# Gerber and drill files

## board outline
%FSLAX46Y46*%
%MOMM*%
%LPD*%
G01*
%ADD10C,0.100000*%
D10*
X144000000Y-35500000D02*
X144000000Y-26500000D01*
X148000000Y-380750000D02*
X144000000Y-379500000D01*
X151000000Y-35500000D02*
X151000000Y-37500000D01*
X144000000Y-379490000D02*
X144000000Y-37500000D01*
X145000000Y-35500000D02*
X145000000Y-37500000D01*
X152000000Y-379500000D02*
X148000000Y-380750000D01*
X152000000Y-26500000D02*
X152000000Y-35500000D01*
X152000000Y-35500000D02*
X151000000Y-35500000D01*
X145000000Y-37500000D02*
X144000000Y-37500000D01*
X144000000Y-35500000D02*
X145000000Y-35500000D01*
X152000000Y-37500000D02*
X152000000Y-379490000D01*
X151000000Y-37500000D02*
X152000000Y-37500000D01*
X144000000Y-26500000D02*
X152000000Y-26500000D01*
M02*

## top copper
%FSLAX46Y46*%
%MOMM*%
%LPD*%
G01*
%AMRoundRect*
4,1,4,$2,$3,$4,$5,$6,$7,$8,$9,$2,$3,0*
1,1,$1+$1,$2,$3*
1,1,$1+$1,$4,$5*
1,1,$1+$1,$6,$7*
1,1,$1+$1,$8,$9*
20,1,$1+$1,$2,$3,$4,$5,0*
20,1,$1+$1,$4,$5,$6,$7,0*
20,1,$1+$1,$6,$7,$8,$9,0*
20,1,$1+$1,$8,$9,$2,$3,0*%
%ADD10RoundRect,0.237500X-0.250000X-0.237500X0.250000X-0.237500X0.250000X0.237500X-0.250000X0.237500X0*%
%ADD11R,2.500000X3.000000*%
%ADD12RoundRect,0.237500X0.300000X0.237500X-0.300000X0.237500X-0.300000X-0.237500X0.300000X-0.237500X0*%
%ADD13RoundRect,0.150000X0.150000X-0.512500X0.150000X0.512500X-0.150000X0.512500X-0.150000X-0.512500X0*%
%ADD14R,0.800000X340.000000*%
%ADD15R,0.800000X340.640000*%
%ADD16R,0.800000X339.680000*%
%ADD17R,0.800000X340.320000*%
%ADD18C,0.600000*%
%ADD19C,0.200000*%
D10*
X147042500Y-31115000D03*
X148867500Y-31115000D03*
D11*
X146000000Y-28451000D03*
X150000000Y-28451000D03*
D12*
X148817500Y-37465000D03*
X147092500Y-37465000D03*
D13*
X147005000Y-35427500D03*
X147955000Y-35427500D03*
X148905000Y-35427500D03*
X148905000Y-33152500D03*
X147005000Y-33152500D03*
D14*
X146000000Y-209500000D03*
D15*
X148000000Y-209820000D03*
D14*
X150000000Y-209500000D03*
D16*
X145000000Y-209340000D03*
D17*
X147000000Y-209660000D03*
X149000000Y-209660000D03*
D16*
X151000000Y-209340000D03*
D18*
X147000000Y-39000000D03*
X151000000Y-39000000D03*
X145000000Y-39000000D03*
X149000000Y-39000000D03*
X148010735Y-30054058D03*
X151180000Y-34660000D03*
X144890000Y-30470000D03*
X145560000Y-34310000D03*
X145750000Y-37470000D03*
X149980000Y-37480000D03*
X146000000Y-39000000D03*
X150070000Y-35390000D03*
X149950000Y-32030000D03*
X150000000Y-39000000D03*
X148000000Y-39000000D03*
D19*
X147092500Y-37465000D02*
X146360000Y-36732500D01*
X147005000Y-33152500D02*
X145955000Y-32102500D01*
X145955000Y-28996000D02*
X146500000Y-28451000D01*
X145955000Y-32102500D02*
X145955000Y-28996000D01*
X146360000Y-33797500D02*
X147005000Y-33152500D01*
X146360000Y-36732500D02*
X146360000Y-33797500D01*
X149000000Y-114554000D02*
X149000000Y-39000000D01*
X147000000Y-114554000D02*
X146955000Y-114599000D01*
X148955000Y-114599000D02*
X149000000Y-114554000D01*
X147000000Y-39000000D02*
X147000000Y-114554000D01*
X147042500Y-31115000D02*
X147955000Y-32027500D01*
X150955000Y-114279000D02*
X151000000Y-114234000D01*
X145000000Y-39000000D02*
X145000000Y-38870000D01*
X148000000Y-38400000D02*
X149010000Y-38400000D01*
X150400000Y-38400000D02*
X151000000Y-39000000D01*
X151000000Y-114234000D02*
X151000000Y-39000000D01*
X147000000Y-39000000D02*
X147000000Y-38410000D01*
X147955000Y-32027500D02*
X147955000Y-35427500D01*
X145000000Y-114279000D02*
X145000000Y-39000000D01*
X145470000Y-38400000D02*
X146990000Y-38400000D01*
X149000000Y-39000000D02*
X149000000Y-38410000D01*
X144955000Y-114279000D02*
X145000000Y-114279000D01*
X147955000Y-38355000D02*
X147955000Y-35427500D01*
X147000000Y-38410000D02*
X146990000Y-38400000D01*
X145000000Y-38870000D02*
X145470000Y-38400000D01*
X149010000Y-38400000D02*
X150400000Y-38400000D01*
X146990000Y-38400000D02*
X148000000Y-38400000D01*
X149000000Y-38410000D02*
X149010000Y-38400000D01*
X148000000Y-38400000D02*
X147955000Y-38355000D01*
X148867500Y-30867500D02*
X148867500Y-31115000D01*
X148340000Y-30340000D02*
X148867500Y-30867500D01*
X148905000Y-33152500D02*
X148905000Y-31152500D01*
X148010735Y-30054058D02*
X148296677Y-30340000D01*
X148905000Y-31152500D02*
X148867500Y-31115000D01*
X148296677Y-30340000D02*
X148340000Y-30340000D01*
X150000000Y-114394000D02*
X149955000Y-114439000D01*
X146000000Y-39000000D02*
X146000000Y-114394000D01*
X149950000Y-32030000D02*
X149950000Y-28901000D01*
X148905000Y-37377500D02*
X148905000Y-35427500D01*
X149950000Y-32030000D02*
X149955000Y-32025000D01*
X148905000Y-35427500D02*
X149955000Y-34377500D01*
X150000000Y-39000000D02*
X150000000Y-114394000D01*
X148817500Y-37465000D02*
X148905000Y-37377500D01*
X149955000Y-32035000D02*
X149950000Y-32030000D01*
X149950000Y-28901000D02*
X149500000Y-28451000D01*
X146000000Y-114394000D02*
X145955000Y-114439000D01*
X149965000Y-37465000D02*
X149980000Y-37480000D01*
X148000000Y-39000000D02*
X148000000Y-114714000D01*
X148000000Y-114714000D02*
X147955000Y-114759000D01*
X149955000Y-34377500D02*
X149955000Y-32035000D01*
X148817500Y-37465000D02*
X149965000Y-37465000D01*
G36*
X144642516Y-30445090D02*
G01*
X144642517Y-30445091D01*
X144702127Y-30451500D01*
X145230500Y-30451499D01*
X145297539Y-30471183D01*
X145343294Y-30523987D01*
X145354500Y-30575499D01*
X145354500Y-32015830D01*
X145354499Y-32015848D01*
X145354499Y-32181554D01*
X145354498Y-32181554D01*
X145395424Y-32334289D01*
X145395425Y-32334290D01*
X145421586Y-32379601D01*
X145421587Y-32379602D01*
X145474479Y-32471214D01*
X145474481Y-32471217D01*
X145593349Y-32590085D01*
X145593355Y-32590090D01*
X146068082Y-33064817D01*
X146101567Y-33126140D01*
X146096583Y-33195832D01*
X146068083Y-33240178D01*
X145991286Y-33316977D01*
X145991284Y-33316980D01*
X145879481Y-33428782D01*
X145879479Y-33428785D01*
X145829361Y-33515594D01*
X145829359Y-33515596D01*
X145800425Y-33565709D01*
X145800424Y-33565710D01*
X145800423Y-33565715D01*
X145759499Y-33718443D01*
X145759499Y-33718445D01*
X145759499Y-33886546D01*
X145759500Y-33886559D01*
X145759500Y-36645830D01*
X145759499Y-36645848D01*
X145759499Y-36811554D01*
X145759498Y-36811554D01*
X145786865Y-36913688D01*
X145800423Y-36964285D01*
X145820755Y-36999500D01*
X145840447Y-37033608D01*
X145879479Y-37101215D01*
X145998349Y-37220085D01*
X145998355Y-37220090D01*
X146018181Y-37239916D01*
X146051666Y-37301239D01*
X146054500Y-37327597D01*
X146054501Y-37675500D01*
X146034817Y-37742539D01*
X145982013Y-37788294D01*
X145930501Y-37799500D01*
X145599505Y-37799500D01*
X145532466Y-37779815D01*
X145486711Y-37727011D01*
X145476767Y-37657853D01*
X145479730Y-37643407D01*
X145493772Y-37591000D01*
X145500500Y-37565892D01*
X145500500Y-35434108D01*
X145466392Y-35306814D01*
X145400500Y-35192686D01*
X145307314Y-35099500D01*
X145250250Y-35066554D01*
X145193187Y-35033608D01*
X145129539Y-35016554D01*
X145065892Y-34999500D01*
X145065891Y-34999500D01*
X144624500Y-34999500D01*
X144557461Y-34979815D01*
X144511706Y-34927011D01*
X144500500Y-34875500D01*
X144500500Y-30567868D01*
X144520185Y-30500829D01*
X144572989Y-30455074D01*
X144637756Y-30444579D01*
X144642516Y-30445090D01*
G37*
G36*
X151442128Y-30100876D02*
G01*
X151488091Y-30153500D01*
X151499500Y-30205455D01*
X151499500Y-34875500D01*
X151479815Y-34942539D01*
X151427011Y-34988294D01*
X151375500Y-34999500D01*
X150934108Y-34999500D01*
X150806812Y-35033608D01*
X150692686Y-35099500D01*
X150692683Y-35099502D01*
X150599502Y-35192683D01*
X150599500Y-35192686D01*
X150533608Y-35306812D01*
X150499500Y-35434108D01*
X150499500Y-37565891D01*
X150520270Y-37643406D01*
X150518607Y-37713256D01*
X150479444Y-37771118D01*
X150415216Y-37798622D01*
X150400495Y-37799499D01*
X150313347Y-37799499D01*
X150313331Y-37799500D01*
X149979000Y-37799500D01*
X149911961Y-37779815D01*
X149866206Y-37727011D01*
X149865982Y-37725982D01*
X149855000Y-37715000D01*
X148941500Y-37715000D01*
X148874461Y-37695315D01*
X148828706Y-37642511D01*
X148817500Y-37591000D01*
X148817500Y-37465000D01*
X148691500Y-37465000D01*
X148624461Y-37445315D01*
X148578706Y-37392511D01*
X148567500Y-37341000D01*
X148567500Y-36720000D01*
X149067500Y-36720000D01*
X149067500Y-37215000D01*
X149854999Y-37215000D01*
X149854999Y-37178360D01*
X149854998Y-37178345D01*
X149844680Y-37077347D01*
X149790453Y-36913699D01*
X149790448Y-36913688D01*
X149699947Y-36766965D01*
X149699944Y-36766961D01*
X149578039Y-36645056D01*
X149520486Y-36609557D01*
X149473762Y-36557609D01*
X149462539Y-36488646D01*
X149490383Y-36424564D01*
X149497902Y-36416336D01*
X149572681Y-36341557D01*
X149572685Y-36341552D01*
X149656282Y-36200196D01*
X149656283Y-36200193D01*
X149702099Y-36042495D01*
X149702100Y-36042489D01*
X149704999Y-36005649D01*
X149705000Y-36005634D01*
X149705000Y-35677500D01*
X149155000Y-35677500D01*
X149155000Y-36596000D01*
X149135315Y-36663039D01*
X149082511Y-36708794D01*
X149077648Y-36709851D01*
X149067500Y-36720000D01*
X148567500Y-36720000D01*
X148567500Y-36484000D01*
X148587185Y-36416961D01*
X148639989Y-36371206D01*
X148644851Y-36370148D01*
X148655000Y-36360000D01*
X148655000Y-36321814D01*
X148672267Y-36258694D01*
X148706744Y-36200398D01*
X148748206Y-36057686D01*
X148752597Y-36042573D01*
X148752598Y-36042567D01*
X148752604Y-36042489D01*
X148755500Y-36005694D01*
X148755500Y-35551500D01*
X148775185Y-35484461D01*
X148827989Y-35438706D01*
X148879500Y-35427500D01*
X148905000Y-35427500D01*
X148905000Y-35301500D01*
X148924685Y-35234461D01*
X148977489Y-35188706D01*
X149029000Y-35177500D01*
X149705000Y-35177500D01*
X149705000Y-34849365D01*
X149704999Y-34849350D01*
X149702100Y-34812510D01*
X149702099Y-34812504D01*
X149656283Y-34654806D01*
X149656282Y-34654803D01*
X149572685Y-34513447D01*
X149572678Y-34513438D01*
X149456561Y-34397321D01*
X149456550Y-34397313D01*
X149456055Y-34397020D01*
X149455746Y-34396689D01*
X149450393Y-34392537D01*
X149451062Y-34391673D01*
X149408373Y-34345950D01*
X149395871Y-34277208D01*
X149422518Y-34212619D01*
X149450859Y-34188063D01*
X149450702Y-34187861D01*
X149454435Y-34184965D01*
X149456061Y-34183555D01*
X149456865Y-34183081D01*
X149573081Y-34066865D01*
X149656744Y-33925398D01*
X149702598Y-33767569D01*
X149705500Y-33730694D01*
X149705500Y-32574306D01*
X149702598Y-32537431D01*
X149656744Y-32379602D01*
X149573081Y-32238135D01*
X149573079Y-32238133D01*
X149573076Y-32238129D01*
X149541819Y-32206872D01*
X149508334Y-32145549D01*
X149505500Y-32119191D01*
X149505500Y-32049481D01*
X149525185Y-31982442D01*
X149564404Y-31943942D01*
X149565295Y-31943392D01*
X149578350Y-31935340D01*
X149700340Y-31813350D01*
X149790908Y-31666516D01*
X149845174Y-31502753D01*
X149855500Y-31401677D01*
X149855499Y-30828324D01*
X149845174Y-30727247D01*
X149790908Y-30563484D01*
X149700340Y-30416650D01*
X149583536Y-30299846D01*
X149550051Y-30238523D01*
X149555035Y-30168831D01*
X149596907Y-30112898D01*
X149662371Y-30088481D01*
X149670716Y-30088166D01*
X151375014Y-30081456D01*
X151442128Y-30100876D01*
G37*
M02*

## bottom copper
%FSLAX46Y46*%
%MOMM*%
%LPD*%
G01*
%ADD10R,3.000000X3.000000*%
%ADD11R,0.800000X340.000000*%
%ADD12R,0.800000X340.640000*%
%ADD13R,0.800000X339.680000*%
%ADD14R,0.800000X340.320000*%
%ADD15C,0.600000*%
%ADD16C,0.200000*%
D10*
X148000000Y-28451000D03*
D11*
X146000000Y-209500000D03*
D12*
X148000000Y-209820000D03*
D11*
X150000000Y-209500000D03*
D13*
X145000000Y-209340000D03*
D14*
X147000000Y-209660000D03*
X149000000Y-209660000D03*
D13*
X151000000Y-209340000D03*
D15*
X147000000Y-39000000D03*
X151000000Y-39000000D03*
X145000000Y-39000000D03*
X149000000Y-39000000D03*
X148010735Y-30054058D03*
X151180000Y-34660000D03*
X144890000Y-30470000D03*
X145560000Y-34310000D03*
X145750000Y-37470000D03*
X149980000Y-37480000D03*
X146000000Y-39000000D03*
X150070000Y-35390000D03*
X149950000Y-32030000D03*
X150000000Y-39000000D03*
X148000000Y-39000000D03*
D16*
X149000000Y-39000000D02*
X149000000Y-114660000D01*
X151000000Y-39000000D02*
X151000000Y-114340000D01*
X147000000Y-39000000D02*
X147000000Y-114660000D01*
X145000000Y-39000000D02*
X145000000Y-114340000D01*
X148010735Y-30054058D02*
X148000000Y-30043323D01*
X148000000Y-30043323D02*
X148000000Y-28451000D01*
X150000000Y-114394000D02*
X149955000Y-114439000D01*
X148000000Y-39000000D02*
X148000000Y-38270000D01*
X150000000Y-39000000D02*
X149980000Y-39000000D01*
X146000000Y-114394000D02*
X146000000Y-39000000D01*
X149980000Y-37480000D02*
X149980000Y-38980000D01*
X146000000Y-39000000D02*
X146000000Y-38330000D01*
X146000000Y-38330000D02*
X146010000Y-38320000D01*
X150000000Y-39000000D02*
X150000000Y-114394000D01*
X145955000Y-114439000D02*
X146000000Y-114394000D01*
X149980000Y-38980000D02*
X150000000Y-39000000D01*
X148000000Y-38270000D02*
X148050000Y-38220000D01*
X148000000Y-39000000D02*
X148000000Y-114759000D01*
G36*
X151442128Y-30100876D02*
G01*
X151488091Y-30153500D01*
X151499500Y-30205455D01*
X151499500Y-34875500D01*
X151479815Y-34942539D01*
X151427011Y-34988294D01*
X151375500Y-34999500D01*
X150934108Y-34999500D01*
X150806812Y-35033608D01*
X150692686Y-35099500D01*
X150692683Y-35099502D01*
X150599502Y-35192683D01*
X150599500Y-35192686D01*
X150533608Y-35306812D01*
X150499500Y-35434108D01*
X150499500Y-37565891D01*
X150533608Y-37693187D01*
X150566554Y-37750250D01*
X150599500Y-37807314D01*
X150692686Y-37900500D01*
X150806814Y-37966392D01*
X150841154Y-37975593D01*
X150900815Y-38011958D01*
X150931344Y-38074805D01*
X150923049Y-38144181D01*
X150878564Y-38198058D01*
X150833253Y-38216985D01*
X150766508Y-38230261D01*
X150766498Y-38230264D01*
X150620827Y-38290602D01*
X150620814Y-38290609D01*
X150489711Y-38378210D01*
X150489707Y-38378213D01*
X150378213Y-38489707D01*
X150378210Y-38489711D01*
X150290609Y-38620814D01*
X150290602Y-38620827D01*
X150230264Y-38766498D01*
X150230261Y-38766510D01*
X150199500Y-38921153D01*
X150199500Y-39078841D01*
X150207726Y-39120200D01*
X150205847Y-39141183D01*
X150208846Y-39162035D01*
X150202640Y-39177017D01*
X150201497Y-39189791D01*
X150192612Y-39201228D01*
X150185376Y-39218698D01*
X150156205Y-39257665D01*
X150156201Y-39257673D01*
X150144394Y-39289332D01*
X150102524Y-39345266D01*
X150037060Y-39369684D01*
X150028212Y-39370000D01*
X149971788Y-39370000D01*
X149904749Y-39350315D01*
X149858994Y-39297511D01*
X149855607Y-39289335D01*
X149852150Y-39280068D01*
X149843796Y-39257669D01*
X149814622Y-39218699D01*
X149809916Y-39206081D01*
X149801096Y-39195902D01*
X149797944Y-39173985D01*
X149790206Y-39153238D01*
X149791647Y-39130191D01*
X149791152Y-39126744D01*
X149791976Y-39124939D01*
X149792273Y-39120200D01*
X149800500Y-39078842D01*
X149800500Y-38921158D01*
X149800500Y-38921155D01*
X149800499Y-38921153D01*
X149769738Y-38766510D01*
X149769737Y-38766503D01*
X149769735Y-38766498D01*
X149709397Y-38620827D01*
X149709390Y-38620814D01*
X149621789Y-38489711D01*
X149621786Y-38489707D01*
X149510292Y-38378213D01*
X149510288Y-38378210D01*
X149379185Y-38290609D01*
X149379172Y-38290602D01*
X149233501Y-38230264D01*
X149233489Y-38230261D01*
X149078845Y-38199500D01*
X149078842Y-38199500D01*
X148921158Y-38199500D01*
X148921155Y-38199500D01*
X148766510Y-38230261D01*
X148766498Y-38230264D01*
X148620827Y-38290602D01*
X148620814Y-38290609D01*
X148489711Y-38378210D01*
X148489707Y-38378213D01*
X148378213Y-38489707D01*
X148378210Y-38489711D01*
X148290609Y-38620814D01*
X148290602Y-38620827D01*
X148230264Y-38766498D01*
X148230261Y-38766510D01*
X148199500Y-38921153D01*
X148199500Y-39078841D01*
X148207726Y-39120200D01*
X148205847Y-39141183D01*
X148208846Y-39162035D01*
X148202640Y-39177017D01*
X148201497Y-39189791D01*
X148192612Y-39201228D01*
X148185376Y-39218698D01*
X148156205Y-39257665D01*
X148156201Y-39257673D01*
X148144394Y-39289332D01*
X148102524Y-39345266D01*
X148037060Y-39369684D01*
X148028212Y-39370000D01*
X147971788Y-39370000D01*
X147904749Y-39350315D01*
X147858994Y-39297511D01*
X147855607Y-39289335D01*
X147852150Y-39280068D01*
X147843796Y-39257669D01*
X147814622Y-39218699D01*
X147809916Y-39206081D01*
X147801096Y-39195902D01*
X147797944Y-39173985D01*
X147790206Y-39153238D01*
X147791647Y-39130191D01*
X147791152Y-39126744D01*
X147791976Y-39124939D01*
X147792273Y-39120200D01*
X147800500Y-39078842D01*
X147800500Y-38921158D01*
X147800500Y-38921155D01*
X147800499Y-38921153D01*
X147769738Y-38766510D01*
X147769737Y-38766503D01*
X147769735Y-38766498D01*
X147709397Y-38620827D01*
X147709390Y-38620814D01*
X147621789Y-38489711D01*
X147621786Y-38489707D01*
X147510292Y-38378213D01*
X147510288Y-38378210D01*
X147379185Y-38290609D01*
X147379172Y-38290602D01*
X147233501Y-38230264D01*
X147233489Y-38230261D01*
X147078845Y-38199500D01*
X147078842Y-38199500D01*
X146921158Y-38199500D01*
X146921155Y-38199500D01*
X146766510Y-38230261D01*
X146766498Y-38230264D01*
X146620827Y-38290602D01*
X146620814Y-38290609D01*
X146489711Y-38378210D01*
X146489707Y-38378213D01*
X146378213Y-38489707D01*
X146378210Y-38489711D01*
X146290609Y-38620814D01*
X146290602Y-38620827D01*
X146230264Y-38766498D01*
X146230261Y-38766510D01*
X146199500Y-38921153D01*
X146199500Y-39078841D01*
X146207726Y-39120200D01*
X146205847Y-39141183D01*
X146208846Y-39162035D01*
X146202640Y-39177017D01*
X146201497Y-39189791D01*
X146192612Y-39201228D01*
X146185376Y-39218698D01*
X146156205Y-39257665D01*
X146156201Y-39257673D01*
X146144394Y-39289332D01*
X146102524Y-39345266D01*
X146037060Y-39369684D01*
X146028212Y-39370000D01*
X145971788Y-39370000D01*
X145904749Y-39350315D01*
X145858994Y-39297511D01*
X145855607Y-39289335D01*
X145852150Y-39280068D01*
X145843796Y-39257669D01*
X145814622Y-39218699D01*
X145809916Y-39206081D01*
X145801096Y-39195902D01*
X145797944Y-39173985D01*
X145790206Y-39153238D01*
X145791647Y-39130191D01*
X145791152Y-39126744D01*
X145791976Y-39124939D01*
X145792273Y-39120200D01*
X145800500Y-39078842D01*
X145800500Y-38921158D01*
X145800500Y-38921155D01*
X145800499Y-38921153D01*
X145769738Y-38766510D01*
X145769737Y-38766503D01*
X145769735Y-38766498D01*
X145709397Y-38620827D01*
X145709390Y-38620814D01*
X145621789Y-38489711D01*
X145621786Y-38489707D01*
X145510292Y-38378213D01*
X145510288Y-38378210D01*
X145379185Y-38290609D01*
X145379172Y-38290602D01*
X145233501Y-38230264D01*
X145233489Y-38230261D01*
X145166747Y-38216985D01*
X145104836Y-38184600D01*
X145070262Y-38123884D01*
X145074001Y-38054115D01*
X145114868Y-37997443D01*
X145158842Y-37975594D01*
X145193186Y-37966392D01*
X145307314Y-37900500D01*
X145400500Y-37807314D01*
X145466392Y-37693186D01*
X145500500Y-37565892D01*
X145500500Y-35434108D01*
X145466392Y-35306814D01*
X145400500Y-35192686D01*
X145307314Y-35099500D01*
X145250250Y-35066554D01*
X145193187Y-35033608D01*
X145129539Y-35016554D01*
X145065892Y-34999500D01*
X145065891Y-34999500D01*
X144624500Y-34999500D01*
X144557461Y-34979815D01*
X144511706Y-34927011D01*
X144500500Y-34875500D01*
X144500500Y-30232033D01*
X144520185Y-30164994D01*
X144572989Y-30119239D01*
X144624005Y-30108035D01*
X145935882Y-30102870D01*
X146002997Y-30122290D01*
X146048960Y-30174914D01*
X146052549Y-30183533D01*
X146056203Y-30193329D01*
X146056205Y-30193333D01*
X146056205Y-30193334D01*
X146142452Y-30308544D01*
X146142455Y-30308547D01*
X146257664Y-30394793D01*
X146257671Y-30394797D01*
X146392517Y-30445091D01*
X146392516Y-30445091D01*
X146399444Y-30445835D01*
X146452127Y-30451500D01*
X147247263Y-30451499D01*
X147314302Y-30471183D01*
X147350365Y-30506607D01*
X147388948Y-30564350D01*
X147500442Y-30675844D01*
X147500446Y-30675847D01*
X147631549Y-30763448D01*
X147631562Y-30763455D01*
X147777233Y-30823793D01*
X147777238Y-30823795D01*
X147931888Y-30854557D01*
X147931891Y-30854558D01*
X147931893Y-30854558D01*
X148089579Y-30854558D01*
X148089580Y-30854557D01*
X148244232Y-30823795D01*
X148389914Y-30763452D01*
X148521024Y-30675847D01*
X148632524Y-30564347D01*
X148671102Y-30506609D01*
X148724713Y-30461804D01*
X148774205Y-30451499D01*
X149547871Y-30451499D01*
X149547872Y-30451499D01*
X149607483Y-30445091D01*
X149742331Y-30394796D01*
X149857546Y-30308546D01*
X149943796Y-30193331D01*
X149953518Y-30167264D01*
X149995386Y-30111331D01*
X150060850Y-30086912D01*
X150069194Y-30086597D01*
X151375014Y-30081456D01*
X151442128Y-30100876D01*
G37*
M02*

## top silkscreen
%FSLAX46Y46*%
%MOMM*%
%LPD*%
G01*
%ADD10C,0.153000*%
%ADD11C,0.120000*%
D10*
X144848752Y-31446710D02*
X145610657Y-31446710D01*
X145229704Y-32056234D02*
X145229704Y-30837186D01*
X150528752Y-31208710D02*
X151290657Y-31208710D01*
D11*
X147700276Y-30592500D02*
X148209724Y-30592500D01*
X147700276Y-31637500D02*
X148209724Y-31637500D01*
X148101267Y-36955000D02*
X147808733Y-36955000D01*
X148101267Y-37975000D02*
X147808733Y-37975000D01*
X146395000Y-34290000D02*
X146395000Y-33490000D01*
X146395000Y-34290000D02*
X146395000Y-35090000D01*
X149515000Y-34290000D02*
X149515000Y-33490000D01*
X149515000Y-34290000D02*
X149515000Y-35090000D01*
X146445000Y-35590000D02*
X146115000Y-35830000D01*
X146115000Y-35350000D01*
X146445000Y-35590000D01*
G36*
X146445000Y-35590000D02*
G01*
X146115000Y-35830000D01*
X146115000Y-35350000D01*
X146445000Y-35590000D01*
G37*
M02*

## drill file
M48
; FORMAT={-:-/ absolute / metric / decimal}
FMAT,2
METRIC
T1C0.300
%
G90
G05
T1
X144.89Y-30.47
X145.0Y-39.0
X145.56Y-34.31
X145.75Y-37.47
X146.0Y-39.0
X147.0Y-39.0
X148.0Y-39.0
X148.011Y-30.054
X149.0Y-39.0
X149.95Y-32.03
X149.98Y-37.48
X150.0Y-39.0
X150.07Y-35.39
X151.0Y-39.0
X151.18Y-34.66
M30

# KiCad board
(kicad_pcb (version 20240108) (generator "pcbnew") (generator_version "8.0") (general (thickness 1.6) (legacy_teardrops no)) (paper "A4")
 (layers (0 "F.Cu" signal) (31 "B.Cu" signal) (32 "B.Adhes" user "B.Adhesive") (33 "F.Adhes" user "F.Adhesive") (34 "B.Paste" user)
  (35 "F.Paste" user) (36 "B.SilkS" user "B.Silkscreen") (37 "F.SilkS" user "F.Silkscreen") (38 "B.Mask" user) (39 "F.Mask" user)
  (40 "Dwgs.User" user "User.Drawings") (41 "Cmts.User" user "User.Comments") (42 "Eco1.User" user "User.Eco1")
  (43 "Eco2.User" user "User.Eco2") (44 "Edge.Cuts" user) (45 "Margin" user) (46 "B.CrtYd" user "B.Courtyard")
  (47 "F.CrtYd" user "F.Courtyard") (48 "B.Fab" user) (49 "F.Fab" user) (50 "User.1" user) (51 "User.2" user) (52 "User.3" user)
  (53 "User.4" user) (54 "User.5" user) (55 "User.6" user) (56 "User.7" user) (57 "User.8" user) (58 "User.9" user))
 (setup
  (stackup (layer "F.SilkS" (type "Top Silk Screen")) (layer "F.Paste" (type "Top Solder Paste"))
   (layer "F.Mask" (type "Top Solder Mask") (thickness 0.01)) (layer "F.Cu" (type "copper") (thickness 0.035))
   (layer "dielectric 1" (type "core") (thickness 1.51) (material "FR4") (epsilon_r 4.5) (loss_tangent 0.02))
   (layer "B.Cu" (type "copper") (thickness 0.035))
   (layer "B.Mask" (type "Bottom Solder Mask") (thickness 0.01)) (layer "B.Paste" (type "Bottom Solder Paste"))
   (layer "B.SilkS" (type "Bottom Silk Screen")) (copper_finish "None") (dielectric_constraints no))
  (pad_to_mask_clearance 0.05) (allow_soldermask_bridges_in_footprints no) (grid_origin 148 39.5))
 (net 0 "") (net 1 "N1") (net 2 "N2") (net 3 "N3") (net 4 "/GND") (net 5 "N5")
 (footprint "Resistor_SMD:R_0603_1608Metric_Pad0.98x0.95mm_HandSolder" (layer "F.Cu") (at 147.955 31.115)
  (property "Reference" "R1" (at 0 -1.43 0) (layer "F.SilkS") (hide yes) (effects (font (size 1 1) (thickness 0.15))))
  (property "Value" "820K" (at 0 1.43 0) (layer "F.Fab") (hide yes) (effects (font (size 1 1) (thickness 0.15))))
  (fp_line (start -0.254724 -0.5225) (end 0.254724 -0.5225) (stroke (width 0.12) (type solid)) (layer "F.SilkS"))
  (fp_line (start -0.254724 0.5225) (end 0.254724 0.5225) (stroke (width 0.12) (type solid)) (layer "F.SilkS"))
  (pad "1" smd roundrect (at -0.9125 0) (size 0.975 0.95) (layers "F.Cu" "F.Paste" "F.Mask") (roundrect_rratio 0.25) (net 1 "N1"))
  (pad "2" smd roundrect (at 0.9125 0) (size 0.975 0.95) (layers "F.Cu" "F.Paste" "F.Mask") (roundrect_rratio 0.25) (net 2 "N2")))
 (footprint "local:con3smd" (layer "F.Cu") (at 148 28.451)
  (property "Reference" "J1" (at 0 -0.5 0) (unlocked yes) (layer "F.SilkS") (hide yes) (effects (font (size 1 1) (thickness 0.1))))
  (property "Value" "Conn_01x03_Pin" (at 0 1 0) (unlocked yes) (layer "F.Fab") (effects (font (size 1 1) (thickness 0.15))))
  (pad "1" smd rect (at -2 0) (size 2.5 3) (layers "F.Cu" "F.Paste" "F.Mask") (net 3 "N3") (thermal_bridge_angle 45))
  (pad "2" smd rect (at 0 0) (size 3 3) (layers "B.Cu" "B.Paste" "B.Mask") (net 2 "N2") (thermal_bridge_angle 45))
  (pad "3" smd rect (at 2 0) (size 2.5 3) (layers "F.Cu" "F.Paste" "F.Mask") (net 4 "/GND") (thermal_bridge_angle 45)))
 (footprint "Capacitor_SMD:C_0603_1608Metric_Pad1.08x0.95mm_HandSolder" (layer "F.Cu") (at 147.955 37.465 180)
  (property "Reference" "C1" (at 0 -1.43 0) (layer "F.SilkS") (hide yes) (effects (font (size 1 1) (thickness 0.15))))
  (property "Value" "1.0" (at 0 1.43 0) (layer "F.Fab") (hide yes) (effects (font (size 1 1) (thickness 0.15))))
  (fp_line (start -0.146267 0.51) (end 0.146267 0.51) (stroke (width 0.12) (type solid)) (layer "F.SilkS"))
  (fp_line (start -0.146267 -0.51) (end 0.146267 -0.51) (stroke (width 0.12) (type solid)) (layer "F.SilkS"))
  (pad "1" smd roundrect (at -0.8625 0 180) (size 1.075 0.95) (layers "F.Cu" "F.Paste" "F.Mask") (roundrect_rratio 0.25) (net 4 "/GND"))
  (pad "2" smd roundrect (at 0.8625 0 180) (size 1.075 0.95) (layers "F.Cu" "F.Paste" "F.Mask") (roundrect_rratio 0.25) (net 3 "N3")))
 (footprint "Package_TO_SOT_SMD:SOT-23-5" (layer "F.Cu") (at 147.955 34.29 90)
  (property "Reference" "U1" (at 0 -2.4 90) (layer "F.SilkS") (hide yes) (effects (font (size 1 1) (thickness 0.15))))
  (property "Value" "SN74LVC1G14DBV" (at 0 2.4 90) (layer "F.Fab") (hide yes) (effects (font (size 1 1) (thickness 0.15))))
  (fp_line (start 0 -1.56) (end 0.8 -1.56) (stroke (width 0.12) (type solid)) (layer "F.SilkS"))
  (fp_line (start 0 -1.56) (end -0.8 -1.56) (stroke (width 0.12) (type solid)) (layer "F.SilkS"))
  (fp_line (start 0 1.56) (end 0.8 1.56) (stroke (width 0.12) (type solid)) (layer "F.SilkS"))
  (fp_line (start 0 1.56) (end -0.8 1.56) (stroke (width 0.12) (type solid)) (layer "F.SilkS"))
  (fp_poly
   (pts (xy -1.3 -1.51) (xy -1.54 -1.84) (xy -1.06 -1.84) (xy -1.3 -1.51)) (stroke (width 0.12) (type solid)) (fill solid) (layer "F.SilkS"))
  (pad "1" smd roundrect (at -1.1375 -0.95 90) (size 1.325 0.6) (layers "F.Cu" "F.Paste" "F.Mask") (roundrect_rratio 0.25) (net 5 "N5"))
  (pad "2" smd roundrect (at -1.1375 0 90) (size 1.325 0.6) (layers "F.Cu" "F.Paste" "F.Mask") (roundrect_rratio 0.25) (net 1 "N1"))
  (pad "3" smd roundrect (at -1.1375 0.95 90) (size 1.325 0.6) (layers "F.Cu" "F.Paste" "F.Mask") (roundrect_rratio 0.25) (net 4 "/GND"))
  (pad "4" smd roundrect (at 1.1375 0.95 90) (size 1.325 0.6) (layers "F.Cu" "F.Paste" "F.Mask") (roundrect_rratio 0.25) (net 2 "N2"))
  (pad "5" smd roundrect (at 1.1375 -0.95 90) (size 1.325 0.6) (layers "F.Cu" "F.Paste" "F.Mask") (roundrect_rratio 0.25) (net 3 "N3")))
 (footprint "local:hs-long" (layer "F.Cu") (at 148 39.5)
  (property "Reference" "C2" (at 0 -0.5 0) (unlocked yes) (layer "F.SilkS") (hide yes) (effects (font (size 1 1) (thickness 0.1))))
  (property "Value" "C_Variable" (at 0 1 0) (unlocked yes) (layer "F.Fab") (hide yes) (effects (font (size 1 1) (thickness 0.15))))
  (pad "1" smd rect (at -2 170) (size 0.8 340) (layers "F.Cu") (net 4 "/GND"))
  (pad "1" smd rect (at -2 170) (size 0.8 340) (layers "B.Cu") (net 4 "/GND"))
  (pad "1" smd rect (at 0 170.32) (size 0.8 340.64) (layers "F.Cu") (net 4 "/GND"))
  (pad "1" smd rect (at 0 170.32) (size 0.8 340.64) (layers "B.Cu") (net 4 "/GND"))
  (pad "1" smd rect (at 2 170) (size 0.8 340) (layers "F.Cu") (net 4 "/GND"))
  (pad "1" smd rect (at 2 170) (size 0.8 340) (layers "B.Cu") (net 4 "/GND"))
  (pad "2" smd rect (at -3 169.84) (size 0.8 339.68) (layers "F.Cu") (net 1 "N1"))
  (pad "2" smd rect (at -3 169.84) (size 0.8 339.68) (layers "B.Cu") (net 1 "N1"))
  (pad "2" smd rect (at -1 170.16) (size 0.8 340.32) (layers "F.Cu") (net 1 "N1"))
  (pad "2" smd rect (at -1 170.16) (size 0.8 340.32) (layers "B.Cu") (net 1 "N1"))
  (pad "2" smd rect (at 1 170.16) (size 0.8 340.32) (layers "F.Cu") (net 1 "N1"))
  (pad "2" smd rect (at 1 170.16) (size 0.8 340.32) (layers "B.Cu") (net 1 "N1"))
  (pad "2" smd rect (at 3 169.84) (size 0.8 339.68) (layers "F.Cu") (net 1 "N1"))
  (pad "2" smd rect (at 3 169.84) (size 0.8 339.68) (layers "B.Cu") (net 1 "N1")))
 (gr_line (start 144 35.5) (end 144 26.5) (stroke (width 0.1) (type default)) (layer "Edge.Cuts"))
 (gr_line (start 148 380.75) (end 144 379.5) (stroke (width 0.1) (type default)) (layer "Edge.Cuts"))
 (gr_line (start 151 35.5) (end 151 37.5) (stroke (width 0.1) (type default)) (layer "Edge.Cuts"))
 (gr_line (start 144 379.49) (end 144 37.5) (stroke (width 0.1) (type default)) (layer "Edge.Cuts"))
 (gr_line (start 145 35.5) (end 145 37.5) (stroke (width 0.1) (type default)) (layer "Edge.Cuts"))
 (gr_line (start 152 379.5) (end 148 380.75) (stroke (width 0.1) (type default)) (layer "Edge.Cuts"))
 (gr_line (start 152 26.5) (end 152 35.5) (stroke (width 0.1) (type default)) (layer "Edge.Cuts"))
 (gr_line (start 152 35.5) (end 151 35.5) (stroke (width 0.1) (type default)) (layer "Edge.Cuts"))
 (gr_line (start 145 37.5) (end 144 37.5) (stroke (width 0.1) (type default)) (layer "Edge.Cuts"))
 (gr_line (start 144 35.5) (end 145 35.5) (stroke (width 0.1) (type default)) (layer "Edge.Cuts"))
 (gr_line (start 152 37.5) (end 152 379.49) (stroke (width 0.1) (type default)) (layer "Edge.Cuts"))
 (gr_line (start 151 37.5) (end 152 37.5) (stroke (width 0.1) (type default)) (layer "Edge.Cuts"))
 (gr_line (start 144 26.5) (end 152 26.5) (stroke (width 0.1) (type default)) (layer "Edge.Cuts"))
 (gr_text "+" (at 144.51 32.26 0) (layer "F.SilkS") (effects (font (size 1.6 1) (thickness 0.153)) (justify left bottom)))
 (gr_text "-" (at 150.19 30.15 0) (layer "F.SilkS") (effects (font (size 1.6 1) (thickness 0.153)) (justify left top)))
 (segment (start 147.0925 37.465) (end 146.36 36.7325) (width 0.2) (layer "F.Cu") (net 3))
 (segment (start 147.005 33.1525) (end 145.955 32.1025) (width 0.2) (layer "F.Cu") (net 3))
 (segment (start 145.955 28.996) (end 146.5 28.451) (width 0.2) (layer "F.Cu") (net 3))
 (segment (start 145.955 32.1025) (end 145.955 28.996) (width 0.2) (layer "F.Cu") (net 3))
 (segment (start 146.36 33.7975) (end 147.005 33.1525) (width 0.2) (layer "F.Cu") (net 3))
 (segment (start 146.36 36.7325) (end 146.36 33.7975) (width 0.2) (layer "F.Cu") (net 3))
 (segment (start 149 114.554) (end 149 39) (width 0.2) (layer "F.Cu") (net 1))
 (segment (start 147 114.554) (end 146.955 114.599) (width 0.2) (layer "F.Cu") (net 1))
 (segment (start 148.955 114.599) (end 149 114.554) (width 0.2) (layer "F.Cu") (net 1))
 (segment (start 147 39) (end 147 114.554) (width 0.2) (layer "F.Cu") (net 1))
 (segment (start 147.0425 31.115) (end 147.955 32.0275) (width 0.2) (layer "F.Cu") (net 1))
 (segment (start 150.955 114.279) (end 151 114.234) (width 0.2) (layer "F.Cu") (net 1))
 (segment (start 145 39) (end 145 38.87) (width 0.2) (layer "F.Cu") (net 1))
 (segment (start 148 38.4) (end 149.01 38.4) (width 0.2) (layer "F.Cu") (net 1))
 (segment (start 150.4 38.4) (end 151 39) (width 0.2) (layer "F.Cu") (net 1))
 (segment (start 151 114.234) (end 151 39) (width 0.2) (layer "F.Cu") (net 1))
 (segment (start 147 39) (end 147 38.41) (width 0.2) (layer "F.Cu") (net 1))
 (segment (start 147.955 32.0275) (end 147.955 35.4275) (width 0.2) (layer "F.Cu") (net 1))
 (segment (start 145 114.279) (end 145 39) (width 0.2) (layer "F.Cu") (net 1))
 (segment (start 145.47 38.4) (end 146.99 38.4) (width 0.2) (layer "F.Cu") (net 1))
 (segment (start 149 39) (end 149 38.41) (width 0.2) (layer "F.Cu") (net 1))
 (segment (start 144.955 114.279) (end 145 114.279) (width 0.2) (layer "F.Cu") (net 1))
 (segment (start 147.955 38.355) (end 147.955 35.4275) (width 0.2) (layer "F.Cu") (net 1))
 (segment (start 147 38.41) (end 146.99 38.4) (width 0.2) (layer "F.Cu") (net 1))
 (segment (start 145 38.87) (end 145.47 38.4) (width 0.2) (layer "F.Cu") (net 1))
 (segment (start 149.01 38.4) (end 150.4 38.4) (width 0.2) (layer "F.Cu") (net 1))
 (segment (start 146.99 38.4) (end 148 38.4) (width 0.2) (layer "F.Cu") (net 1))
 (segment (start 149 38.41) (end 149.01 38.4) (width 0.2) (layer "F.Cu") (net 1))
 (segment (start 148 38.4) (end 147.955 38.355) (width 0.2) (layer "F.Cu") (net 1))
 (via (at 147 39) (size 0.6) (drill 0.3) (layers "F.Cu" "B.Cu") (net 1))
 (via (at 151 39) (size 0.6) (drill 0.3) (layers "F.Cu" "B.Cu") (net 1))
 (via (at 145 39) (size 0.6) (drill 0.3) (layers "F.Cu" "B.Cu") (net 1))
 (via (at 149 39) (size 0.6) (drill 0.3) (layers "F.Cu" "B.Cu") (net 1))
 (segment (start 149 39) (end 149 114.66) (width 0.2) (layer "B.Cu") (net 1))
 (segment (start 151 39) (end 151 114.34) (width 0.2) (layer "B.Cu") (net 1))
 (segment (start 147 39) (end 147 114.66) (width 0.2) (layer "B.Cu") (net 1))
 (segment (start 145 39) (end 145 114.34) (width 0.2) (layer "B.Cu") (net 1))
 (segment (start 148.8675 30.8675) (end 148.8675 31.115) (width 0.2) (layer "F.Cu") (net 2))
 (segment (start 148.34 30.34) (end 148.8675 30.8675) (width 0.2) (layer "F.Cu") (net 2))
 (segment (start 148.905 33.1525) (end 148.905 31.1525) (width 0.2) (layer "F.Cu") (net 2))
 (segment (start 148.010735 30.054058) (end 148.296677 30.34) (width 0.2) (layer "F.Cu") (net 2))
 (segment (start 148.905 31.1525) (end 148.8675 31.115) (width 0.2) (layer "F.Cu") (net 2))
 (segment (start 148.296677 30.34) (end 148.34 30.34) (width 0.2) (layer "F.Cu") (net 2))
 (via (at 148.010735 30.054058) (size 0.6) (drill 0.3) (layers "F.Cu" "B.Cu") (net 2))
 (segment (start 148.010735 30.054058) (end 148 30.043323) (width 0.2) (layer "B.Cu") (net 2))
 (segment (start 148 30.043323) (end 148 28.451) (width 0.2) (layer "B.Cu") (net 2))
 (segment (start 150 114.394) (end 149.955 114.439) (width 0.2) (layer "F.Cu") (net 4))
 (segment (start 146 39) (end 146 114.394) (width 0.2) (layer "F.Cu") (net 4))
 (segment (start 149.95 32.03) (end 149.95 28.901) (width 0.2) (layer "F.Cu") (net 4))
 (segment (start 148.905 37.3775) (end 148.905 35.4275) (width 0.2) (layer "F.Cu") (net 4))
 (segment (start 149.95 32.03) (end 149.955 32.025) (width 0.2) (layer "F.Cu") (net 4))
 (segment (start 148.905 35.4275) (end 149.955 34.3775) (width 0.2) (layer "F.Cu") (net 4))
 (segment (start 150 39) (end 150 114.394) (width 0.2) (layer "F.Cu") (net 4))
 (segment (start 148.8175 37.465) (end 148.905 37.3775) (width 0.2) (layer "F.Cu") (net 4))
 (segment (start 149.955 32.035) (end 149.95 32.03) (width 0.2) (layer "F.Cu") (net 4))
 (segment (start 149.95 28.901) (end 149.5 28.451) (width 0.2) (layer "F.Cu") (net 4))
 (segment (start 146 114.394) (end 145.955 114.439) (width 0.2) (layer "F.Cu") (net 4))
 (segment (start 149.965 37.465) (end 149.98 37.48) (width 0.2) (layer "F.Cu") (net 4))
 (segment (start 148 39) (end 148 114.714) (width 0.2) (layer "F.Cu") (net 4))
 (segment (start 148 114.714) (end 147.955 114.759) (width 0.2) (layer "F.Cu") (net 4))
 (segment (start 149.955 34.3775) (end 149.955 32.035) (width 0.2) (layer "F.Cu") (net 4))
 (segment (start 148.8175 37.465) (end 149.965 37.465) (width 0.2) (layer "F.Cu") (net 4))
 (via (at 151.18 34.66) (size 0.6) (drill 0.3) (layers "F.Cu" "B.Cu") (free yes) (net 4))
 (via (at 144.89 30.47) (size 0.6) (drill 0.3) (layers "F.Cu" "B.Cu") (free yes) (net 4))
 (via (at 145.56 34.31) (size 0.6) (drill 0.3) (layers "F.Cu" "B.Cu") (free yes) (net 4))
 (via (at 145.75 37.47) (size 0.6) (drill 0.3) (layers "F.Cu" "B.Cu") (free yes) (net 4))
 (via (at 149.98 37.48) (size 0.6) (drill 0.3) (layers "F.Cu" "B.Cu") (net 4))
 (via (at 146 39) (size 0.6) (drill 0.3) (layers "F.Cu" "B.Cu") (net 4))
 (via (at 150.07 35.39) (size 0.6) (drill 0.3) (layers "F.Cu" "B.Cu") (free yes) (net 4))
 (via (at 149.95 32.03) (size 0.6) (drill 0.3) (layers "F.Cu" "B.Cu") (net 4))
 (via (at 150 39) (size 0.6) (drill 0.3) (layers "F.Cu" "B.Cu") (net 4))
 (via (at 148 39) (size 0.6) (drill 0.3) (layers "F.Cu" "B.Cu") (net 4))
 (segment (start 150 114.394) (end 149.955 114.439) (width 0.2) (layer "B.Cu") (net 4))
 (segment (start 148 39) (end 148 38.27) (width 0.2) (layer "B.Cu") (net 4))
 (segment (start 150 39) (end 149.98 39) (width 0.2) (layer "B.Cu") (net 4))
 (segment (start 146 114.394) (end 146 39) (width 0.2) (layer "B.Cu") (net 4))
 (segment (start 149.98 37.48) (end 149.98 38.98) (width 0.2) (layer "B.Cu") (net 4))
 (segment (start 146 39) (end 146 38.33) (width 0.2) (layer "B.Cu") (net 4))
 (segment (start 146 38.33) (end 146.01 38.32) (width 0.2) (layer "B.Cu") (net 4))
 (segment (start 150 39) (end 150 114.394) (width 0.2) (layer "B.Cu") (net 4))
 (segment (start 145.955 114.439) (end 146 114.394) (width 0.2) (layer "B.Cu") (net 4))
 (segment (start 149.98 38.98) (end 150 39) (width 0.2) (layer "B.Cu") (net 4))
 (segment (start 148 38.27) (end 148.05 38.22) (width 0.2) (layer "B.Cu") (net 4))
 (segment (start 148 39) (end 148 114.759) (width 0.2) (layer "B.Cu") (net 4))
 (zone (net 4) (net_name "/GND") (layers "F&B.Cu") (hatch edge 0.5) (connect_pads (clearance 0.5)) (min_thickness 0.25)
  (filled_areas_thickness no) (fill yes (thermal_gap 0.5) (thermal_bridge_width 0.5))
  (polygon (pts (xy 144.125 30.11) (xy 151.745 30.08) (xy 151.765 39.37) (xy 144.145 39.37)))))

